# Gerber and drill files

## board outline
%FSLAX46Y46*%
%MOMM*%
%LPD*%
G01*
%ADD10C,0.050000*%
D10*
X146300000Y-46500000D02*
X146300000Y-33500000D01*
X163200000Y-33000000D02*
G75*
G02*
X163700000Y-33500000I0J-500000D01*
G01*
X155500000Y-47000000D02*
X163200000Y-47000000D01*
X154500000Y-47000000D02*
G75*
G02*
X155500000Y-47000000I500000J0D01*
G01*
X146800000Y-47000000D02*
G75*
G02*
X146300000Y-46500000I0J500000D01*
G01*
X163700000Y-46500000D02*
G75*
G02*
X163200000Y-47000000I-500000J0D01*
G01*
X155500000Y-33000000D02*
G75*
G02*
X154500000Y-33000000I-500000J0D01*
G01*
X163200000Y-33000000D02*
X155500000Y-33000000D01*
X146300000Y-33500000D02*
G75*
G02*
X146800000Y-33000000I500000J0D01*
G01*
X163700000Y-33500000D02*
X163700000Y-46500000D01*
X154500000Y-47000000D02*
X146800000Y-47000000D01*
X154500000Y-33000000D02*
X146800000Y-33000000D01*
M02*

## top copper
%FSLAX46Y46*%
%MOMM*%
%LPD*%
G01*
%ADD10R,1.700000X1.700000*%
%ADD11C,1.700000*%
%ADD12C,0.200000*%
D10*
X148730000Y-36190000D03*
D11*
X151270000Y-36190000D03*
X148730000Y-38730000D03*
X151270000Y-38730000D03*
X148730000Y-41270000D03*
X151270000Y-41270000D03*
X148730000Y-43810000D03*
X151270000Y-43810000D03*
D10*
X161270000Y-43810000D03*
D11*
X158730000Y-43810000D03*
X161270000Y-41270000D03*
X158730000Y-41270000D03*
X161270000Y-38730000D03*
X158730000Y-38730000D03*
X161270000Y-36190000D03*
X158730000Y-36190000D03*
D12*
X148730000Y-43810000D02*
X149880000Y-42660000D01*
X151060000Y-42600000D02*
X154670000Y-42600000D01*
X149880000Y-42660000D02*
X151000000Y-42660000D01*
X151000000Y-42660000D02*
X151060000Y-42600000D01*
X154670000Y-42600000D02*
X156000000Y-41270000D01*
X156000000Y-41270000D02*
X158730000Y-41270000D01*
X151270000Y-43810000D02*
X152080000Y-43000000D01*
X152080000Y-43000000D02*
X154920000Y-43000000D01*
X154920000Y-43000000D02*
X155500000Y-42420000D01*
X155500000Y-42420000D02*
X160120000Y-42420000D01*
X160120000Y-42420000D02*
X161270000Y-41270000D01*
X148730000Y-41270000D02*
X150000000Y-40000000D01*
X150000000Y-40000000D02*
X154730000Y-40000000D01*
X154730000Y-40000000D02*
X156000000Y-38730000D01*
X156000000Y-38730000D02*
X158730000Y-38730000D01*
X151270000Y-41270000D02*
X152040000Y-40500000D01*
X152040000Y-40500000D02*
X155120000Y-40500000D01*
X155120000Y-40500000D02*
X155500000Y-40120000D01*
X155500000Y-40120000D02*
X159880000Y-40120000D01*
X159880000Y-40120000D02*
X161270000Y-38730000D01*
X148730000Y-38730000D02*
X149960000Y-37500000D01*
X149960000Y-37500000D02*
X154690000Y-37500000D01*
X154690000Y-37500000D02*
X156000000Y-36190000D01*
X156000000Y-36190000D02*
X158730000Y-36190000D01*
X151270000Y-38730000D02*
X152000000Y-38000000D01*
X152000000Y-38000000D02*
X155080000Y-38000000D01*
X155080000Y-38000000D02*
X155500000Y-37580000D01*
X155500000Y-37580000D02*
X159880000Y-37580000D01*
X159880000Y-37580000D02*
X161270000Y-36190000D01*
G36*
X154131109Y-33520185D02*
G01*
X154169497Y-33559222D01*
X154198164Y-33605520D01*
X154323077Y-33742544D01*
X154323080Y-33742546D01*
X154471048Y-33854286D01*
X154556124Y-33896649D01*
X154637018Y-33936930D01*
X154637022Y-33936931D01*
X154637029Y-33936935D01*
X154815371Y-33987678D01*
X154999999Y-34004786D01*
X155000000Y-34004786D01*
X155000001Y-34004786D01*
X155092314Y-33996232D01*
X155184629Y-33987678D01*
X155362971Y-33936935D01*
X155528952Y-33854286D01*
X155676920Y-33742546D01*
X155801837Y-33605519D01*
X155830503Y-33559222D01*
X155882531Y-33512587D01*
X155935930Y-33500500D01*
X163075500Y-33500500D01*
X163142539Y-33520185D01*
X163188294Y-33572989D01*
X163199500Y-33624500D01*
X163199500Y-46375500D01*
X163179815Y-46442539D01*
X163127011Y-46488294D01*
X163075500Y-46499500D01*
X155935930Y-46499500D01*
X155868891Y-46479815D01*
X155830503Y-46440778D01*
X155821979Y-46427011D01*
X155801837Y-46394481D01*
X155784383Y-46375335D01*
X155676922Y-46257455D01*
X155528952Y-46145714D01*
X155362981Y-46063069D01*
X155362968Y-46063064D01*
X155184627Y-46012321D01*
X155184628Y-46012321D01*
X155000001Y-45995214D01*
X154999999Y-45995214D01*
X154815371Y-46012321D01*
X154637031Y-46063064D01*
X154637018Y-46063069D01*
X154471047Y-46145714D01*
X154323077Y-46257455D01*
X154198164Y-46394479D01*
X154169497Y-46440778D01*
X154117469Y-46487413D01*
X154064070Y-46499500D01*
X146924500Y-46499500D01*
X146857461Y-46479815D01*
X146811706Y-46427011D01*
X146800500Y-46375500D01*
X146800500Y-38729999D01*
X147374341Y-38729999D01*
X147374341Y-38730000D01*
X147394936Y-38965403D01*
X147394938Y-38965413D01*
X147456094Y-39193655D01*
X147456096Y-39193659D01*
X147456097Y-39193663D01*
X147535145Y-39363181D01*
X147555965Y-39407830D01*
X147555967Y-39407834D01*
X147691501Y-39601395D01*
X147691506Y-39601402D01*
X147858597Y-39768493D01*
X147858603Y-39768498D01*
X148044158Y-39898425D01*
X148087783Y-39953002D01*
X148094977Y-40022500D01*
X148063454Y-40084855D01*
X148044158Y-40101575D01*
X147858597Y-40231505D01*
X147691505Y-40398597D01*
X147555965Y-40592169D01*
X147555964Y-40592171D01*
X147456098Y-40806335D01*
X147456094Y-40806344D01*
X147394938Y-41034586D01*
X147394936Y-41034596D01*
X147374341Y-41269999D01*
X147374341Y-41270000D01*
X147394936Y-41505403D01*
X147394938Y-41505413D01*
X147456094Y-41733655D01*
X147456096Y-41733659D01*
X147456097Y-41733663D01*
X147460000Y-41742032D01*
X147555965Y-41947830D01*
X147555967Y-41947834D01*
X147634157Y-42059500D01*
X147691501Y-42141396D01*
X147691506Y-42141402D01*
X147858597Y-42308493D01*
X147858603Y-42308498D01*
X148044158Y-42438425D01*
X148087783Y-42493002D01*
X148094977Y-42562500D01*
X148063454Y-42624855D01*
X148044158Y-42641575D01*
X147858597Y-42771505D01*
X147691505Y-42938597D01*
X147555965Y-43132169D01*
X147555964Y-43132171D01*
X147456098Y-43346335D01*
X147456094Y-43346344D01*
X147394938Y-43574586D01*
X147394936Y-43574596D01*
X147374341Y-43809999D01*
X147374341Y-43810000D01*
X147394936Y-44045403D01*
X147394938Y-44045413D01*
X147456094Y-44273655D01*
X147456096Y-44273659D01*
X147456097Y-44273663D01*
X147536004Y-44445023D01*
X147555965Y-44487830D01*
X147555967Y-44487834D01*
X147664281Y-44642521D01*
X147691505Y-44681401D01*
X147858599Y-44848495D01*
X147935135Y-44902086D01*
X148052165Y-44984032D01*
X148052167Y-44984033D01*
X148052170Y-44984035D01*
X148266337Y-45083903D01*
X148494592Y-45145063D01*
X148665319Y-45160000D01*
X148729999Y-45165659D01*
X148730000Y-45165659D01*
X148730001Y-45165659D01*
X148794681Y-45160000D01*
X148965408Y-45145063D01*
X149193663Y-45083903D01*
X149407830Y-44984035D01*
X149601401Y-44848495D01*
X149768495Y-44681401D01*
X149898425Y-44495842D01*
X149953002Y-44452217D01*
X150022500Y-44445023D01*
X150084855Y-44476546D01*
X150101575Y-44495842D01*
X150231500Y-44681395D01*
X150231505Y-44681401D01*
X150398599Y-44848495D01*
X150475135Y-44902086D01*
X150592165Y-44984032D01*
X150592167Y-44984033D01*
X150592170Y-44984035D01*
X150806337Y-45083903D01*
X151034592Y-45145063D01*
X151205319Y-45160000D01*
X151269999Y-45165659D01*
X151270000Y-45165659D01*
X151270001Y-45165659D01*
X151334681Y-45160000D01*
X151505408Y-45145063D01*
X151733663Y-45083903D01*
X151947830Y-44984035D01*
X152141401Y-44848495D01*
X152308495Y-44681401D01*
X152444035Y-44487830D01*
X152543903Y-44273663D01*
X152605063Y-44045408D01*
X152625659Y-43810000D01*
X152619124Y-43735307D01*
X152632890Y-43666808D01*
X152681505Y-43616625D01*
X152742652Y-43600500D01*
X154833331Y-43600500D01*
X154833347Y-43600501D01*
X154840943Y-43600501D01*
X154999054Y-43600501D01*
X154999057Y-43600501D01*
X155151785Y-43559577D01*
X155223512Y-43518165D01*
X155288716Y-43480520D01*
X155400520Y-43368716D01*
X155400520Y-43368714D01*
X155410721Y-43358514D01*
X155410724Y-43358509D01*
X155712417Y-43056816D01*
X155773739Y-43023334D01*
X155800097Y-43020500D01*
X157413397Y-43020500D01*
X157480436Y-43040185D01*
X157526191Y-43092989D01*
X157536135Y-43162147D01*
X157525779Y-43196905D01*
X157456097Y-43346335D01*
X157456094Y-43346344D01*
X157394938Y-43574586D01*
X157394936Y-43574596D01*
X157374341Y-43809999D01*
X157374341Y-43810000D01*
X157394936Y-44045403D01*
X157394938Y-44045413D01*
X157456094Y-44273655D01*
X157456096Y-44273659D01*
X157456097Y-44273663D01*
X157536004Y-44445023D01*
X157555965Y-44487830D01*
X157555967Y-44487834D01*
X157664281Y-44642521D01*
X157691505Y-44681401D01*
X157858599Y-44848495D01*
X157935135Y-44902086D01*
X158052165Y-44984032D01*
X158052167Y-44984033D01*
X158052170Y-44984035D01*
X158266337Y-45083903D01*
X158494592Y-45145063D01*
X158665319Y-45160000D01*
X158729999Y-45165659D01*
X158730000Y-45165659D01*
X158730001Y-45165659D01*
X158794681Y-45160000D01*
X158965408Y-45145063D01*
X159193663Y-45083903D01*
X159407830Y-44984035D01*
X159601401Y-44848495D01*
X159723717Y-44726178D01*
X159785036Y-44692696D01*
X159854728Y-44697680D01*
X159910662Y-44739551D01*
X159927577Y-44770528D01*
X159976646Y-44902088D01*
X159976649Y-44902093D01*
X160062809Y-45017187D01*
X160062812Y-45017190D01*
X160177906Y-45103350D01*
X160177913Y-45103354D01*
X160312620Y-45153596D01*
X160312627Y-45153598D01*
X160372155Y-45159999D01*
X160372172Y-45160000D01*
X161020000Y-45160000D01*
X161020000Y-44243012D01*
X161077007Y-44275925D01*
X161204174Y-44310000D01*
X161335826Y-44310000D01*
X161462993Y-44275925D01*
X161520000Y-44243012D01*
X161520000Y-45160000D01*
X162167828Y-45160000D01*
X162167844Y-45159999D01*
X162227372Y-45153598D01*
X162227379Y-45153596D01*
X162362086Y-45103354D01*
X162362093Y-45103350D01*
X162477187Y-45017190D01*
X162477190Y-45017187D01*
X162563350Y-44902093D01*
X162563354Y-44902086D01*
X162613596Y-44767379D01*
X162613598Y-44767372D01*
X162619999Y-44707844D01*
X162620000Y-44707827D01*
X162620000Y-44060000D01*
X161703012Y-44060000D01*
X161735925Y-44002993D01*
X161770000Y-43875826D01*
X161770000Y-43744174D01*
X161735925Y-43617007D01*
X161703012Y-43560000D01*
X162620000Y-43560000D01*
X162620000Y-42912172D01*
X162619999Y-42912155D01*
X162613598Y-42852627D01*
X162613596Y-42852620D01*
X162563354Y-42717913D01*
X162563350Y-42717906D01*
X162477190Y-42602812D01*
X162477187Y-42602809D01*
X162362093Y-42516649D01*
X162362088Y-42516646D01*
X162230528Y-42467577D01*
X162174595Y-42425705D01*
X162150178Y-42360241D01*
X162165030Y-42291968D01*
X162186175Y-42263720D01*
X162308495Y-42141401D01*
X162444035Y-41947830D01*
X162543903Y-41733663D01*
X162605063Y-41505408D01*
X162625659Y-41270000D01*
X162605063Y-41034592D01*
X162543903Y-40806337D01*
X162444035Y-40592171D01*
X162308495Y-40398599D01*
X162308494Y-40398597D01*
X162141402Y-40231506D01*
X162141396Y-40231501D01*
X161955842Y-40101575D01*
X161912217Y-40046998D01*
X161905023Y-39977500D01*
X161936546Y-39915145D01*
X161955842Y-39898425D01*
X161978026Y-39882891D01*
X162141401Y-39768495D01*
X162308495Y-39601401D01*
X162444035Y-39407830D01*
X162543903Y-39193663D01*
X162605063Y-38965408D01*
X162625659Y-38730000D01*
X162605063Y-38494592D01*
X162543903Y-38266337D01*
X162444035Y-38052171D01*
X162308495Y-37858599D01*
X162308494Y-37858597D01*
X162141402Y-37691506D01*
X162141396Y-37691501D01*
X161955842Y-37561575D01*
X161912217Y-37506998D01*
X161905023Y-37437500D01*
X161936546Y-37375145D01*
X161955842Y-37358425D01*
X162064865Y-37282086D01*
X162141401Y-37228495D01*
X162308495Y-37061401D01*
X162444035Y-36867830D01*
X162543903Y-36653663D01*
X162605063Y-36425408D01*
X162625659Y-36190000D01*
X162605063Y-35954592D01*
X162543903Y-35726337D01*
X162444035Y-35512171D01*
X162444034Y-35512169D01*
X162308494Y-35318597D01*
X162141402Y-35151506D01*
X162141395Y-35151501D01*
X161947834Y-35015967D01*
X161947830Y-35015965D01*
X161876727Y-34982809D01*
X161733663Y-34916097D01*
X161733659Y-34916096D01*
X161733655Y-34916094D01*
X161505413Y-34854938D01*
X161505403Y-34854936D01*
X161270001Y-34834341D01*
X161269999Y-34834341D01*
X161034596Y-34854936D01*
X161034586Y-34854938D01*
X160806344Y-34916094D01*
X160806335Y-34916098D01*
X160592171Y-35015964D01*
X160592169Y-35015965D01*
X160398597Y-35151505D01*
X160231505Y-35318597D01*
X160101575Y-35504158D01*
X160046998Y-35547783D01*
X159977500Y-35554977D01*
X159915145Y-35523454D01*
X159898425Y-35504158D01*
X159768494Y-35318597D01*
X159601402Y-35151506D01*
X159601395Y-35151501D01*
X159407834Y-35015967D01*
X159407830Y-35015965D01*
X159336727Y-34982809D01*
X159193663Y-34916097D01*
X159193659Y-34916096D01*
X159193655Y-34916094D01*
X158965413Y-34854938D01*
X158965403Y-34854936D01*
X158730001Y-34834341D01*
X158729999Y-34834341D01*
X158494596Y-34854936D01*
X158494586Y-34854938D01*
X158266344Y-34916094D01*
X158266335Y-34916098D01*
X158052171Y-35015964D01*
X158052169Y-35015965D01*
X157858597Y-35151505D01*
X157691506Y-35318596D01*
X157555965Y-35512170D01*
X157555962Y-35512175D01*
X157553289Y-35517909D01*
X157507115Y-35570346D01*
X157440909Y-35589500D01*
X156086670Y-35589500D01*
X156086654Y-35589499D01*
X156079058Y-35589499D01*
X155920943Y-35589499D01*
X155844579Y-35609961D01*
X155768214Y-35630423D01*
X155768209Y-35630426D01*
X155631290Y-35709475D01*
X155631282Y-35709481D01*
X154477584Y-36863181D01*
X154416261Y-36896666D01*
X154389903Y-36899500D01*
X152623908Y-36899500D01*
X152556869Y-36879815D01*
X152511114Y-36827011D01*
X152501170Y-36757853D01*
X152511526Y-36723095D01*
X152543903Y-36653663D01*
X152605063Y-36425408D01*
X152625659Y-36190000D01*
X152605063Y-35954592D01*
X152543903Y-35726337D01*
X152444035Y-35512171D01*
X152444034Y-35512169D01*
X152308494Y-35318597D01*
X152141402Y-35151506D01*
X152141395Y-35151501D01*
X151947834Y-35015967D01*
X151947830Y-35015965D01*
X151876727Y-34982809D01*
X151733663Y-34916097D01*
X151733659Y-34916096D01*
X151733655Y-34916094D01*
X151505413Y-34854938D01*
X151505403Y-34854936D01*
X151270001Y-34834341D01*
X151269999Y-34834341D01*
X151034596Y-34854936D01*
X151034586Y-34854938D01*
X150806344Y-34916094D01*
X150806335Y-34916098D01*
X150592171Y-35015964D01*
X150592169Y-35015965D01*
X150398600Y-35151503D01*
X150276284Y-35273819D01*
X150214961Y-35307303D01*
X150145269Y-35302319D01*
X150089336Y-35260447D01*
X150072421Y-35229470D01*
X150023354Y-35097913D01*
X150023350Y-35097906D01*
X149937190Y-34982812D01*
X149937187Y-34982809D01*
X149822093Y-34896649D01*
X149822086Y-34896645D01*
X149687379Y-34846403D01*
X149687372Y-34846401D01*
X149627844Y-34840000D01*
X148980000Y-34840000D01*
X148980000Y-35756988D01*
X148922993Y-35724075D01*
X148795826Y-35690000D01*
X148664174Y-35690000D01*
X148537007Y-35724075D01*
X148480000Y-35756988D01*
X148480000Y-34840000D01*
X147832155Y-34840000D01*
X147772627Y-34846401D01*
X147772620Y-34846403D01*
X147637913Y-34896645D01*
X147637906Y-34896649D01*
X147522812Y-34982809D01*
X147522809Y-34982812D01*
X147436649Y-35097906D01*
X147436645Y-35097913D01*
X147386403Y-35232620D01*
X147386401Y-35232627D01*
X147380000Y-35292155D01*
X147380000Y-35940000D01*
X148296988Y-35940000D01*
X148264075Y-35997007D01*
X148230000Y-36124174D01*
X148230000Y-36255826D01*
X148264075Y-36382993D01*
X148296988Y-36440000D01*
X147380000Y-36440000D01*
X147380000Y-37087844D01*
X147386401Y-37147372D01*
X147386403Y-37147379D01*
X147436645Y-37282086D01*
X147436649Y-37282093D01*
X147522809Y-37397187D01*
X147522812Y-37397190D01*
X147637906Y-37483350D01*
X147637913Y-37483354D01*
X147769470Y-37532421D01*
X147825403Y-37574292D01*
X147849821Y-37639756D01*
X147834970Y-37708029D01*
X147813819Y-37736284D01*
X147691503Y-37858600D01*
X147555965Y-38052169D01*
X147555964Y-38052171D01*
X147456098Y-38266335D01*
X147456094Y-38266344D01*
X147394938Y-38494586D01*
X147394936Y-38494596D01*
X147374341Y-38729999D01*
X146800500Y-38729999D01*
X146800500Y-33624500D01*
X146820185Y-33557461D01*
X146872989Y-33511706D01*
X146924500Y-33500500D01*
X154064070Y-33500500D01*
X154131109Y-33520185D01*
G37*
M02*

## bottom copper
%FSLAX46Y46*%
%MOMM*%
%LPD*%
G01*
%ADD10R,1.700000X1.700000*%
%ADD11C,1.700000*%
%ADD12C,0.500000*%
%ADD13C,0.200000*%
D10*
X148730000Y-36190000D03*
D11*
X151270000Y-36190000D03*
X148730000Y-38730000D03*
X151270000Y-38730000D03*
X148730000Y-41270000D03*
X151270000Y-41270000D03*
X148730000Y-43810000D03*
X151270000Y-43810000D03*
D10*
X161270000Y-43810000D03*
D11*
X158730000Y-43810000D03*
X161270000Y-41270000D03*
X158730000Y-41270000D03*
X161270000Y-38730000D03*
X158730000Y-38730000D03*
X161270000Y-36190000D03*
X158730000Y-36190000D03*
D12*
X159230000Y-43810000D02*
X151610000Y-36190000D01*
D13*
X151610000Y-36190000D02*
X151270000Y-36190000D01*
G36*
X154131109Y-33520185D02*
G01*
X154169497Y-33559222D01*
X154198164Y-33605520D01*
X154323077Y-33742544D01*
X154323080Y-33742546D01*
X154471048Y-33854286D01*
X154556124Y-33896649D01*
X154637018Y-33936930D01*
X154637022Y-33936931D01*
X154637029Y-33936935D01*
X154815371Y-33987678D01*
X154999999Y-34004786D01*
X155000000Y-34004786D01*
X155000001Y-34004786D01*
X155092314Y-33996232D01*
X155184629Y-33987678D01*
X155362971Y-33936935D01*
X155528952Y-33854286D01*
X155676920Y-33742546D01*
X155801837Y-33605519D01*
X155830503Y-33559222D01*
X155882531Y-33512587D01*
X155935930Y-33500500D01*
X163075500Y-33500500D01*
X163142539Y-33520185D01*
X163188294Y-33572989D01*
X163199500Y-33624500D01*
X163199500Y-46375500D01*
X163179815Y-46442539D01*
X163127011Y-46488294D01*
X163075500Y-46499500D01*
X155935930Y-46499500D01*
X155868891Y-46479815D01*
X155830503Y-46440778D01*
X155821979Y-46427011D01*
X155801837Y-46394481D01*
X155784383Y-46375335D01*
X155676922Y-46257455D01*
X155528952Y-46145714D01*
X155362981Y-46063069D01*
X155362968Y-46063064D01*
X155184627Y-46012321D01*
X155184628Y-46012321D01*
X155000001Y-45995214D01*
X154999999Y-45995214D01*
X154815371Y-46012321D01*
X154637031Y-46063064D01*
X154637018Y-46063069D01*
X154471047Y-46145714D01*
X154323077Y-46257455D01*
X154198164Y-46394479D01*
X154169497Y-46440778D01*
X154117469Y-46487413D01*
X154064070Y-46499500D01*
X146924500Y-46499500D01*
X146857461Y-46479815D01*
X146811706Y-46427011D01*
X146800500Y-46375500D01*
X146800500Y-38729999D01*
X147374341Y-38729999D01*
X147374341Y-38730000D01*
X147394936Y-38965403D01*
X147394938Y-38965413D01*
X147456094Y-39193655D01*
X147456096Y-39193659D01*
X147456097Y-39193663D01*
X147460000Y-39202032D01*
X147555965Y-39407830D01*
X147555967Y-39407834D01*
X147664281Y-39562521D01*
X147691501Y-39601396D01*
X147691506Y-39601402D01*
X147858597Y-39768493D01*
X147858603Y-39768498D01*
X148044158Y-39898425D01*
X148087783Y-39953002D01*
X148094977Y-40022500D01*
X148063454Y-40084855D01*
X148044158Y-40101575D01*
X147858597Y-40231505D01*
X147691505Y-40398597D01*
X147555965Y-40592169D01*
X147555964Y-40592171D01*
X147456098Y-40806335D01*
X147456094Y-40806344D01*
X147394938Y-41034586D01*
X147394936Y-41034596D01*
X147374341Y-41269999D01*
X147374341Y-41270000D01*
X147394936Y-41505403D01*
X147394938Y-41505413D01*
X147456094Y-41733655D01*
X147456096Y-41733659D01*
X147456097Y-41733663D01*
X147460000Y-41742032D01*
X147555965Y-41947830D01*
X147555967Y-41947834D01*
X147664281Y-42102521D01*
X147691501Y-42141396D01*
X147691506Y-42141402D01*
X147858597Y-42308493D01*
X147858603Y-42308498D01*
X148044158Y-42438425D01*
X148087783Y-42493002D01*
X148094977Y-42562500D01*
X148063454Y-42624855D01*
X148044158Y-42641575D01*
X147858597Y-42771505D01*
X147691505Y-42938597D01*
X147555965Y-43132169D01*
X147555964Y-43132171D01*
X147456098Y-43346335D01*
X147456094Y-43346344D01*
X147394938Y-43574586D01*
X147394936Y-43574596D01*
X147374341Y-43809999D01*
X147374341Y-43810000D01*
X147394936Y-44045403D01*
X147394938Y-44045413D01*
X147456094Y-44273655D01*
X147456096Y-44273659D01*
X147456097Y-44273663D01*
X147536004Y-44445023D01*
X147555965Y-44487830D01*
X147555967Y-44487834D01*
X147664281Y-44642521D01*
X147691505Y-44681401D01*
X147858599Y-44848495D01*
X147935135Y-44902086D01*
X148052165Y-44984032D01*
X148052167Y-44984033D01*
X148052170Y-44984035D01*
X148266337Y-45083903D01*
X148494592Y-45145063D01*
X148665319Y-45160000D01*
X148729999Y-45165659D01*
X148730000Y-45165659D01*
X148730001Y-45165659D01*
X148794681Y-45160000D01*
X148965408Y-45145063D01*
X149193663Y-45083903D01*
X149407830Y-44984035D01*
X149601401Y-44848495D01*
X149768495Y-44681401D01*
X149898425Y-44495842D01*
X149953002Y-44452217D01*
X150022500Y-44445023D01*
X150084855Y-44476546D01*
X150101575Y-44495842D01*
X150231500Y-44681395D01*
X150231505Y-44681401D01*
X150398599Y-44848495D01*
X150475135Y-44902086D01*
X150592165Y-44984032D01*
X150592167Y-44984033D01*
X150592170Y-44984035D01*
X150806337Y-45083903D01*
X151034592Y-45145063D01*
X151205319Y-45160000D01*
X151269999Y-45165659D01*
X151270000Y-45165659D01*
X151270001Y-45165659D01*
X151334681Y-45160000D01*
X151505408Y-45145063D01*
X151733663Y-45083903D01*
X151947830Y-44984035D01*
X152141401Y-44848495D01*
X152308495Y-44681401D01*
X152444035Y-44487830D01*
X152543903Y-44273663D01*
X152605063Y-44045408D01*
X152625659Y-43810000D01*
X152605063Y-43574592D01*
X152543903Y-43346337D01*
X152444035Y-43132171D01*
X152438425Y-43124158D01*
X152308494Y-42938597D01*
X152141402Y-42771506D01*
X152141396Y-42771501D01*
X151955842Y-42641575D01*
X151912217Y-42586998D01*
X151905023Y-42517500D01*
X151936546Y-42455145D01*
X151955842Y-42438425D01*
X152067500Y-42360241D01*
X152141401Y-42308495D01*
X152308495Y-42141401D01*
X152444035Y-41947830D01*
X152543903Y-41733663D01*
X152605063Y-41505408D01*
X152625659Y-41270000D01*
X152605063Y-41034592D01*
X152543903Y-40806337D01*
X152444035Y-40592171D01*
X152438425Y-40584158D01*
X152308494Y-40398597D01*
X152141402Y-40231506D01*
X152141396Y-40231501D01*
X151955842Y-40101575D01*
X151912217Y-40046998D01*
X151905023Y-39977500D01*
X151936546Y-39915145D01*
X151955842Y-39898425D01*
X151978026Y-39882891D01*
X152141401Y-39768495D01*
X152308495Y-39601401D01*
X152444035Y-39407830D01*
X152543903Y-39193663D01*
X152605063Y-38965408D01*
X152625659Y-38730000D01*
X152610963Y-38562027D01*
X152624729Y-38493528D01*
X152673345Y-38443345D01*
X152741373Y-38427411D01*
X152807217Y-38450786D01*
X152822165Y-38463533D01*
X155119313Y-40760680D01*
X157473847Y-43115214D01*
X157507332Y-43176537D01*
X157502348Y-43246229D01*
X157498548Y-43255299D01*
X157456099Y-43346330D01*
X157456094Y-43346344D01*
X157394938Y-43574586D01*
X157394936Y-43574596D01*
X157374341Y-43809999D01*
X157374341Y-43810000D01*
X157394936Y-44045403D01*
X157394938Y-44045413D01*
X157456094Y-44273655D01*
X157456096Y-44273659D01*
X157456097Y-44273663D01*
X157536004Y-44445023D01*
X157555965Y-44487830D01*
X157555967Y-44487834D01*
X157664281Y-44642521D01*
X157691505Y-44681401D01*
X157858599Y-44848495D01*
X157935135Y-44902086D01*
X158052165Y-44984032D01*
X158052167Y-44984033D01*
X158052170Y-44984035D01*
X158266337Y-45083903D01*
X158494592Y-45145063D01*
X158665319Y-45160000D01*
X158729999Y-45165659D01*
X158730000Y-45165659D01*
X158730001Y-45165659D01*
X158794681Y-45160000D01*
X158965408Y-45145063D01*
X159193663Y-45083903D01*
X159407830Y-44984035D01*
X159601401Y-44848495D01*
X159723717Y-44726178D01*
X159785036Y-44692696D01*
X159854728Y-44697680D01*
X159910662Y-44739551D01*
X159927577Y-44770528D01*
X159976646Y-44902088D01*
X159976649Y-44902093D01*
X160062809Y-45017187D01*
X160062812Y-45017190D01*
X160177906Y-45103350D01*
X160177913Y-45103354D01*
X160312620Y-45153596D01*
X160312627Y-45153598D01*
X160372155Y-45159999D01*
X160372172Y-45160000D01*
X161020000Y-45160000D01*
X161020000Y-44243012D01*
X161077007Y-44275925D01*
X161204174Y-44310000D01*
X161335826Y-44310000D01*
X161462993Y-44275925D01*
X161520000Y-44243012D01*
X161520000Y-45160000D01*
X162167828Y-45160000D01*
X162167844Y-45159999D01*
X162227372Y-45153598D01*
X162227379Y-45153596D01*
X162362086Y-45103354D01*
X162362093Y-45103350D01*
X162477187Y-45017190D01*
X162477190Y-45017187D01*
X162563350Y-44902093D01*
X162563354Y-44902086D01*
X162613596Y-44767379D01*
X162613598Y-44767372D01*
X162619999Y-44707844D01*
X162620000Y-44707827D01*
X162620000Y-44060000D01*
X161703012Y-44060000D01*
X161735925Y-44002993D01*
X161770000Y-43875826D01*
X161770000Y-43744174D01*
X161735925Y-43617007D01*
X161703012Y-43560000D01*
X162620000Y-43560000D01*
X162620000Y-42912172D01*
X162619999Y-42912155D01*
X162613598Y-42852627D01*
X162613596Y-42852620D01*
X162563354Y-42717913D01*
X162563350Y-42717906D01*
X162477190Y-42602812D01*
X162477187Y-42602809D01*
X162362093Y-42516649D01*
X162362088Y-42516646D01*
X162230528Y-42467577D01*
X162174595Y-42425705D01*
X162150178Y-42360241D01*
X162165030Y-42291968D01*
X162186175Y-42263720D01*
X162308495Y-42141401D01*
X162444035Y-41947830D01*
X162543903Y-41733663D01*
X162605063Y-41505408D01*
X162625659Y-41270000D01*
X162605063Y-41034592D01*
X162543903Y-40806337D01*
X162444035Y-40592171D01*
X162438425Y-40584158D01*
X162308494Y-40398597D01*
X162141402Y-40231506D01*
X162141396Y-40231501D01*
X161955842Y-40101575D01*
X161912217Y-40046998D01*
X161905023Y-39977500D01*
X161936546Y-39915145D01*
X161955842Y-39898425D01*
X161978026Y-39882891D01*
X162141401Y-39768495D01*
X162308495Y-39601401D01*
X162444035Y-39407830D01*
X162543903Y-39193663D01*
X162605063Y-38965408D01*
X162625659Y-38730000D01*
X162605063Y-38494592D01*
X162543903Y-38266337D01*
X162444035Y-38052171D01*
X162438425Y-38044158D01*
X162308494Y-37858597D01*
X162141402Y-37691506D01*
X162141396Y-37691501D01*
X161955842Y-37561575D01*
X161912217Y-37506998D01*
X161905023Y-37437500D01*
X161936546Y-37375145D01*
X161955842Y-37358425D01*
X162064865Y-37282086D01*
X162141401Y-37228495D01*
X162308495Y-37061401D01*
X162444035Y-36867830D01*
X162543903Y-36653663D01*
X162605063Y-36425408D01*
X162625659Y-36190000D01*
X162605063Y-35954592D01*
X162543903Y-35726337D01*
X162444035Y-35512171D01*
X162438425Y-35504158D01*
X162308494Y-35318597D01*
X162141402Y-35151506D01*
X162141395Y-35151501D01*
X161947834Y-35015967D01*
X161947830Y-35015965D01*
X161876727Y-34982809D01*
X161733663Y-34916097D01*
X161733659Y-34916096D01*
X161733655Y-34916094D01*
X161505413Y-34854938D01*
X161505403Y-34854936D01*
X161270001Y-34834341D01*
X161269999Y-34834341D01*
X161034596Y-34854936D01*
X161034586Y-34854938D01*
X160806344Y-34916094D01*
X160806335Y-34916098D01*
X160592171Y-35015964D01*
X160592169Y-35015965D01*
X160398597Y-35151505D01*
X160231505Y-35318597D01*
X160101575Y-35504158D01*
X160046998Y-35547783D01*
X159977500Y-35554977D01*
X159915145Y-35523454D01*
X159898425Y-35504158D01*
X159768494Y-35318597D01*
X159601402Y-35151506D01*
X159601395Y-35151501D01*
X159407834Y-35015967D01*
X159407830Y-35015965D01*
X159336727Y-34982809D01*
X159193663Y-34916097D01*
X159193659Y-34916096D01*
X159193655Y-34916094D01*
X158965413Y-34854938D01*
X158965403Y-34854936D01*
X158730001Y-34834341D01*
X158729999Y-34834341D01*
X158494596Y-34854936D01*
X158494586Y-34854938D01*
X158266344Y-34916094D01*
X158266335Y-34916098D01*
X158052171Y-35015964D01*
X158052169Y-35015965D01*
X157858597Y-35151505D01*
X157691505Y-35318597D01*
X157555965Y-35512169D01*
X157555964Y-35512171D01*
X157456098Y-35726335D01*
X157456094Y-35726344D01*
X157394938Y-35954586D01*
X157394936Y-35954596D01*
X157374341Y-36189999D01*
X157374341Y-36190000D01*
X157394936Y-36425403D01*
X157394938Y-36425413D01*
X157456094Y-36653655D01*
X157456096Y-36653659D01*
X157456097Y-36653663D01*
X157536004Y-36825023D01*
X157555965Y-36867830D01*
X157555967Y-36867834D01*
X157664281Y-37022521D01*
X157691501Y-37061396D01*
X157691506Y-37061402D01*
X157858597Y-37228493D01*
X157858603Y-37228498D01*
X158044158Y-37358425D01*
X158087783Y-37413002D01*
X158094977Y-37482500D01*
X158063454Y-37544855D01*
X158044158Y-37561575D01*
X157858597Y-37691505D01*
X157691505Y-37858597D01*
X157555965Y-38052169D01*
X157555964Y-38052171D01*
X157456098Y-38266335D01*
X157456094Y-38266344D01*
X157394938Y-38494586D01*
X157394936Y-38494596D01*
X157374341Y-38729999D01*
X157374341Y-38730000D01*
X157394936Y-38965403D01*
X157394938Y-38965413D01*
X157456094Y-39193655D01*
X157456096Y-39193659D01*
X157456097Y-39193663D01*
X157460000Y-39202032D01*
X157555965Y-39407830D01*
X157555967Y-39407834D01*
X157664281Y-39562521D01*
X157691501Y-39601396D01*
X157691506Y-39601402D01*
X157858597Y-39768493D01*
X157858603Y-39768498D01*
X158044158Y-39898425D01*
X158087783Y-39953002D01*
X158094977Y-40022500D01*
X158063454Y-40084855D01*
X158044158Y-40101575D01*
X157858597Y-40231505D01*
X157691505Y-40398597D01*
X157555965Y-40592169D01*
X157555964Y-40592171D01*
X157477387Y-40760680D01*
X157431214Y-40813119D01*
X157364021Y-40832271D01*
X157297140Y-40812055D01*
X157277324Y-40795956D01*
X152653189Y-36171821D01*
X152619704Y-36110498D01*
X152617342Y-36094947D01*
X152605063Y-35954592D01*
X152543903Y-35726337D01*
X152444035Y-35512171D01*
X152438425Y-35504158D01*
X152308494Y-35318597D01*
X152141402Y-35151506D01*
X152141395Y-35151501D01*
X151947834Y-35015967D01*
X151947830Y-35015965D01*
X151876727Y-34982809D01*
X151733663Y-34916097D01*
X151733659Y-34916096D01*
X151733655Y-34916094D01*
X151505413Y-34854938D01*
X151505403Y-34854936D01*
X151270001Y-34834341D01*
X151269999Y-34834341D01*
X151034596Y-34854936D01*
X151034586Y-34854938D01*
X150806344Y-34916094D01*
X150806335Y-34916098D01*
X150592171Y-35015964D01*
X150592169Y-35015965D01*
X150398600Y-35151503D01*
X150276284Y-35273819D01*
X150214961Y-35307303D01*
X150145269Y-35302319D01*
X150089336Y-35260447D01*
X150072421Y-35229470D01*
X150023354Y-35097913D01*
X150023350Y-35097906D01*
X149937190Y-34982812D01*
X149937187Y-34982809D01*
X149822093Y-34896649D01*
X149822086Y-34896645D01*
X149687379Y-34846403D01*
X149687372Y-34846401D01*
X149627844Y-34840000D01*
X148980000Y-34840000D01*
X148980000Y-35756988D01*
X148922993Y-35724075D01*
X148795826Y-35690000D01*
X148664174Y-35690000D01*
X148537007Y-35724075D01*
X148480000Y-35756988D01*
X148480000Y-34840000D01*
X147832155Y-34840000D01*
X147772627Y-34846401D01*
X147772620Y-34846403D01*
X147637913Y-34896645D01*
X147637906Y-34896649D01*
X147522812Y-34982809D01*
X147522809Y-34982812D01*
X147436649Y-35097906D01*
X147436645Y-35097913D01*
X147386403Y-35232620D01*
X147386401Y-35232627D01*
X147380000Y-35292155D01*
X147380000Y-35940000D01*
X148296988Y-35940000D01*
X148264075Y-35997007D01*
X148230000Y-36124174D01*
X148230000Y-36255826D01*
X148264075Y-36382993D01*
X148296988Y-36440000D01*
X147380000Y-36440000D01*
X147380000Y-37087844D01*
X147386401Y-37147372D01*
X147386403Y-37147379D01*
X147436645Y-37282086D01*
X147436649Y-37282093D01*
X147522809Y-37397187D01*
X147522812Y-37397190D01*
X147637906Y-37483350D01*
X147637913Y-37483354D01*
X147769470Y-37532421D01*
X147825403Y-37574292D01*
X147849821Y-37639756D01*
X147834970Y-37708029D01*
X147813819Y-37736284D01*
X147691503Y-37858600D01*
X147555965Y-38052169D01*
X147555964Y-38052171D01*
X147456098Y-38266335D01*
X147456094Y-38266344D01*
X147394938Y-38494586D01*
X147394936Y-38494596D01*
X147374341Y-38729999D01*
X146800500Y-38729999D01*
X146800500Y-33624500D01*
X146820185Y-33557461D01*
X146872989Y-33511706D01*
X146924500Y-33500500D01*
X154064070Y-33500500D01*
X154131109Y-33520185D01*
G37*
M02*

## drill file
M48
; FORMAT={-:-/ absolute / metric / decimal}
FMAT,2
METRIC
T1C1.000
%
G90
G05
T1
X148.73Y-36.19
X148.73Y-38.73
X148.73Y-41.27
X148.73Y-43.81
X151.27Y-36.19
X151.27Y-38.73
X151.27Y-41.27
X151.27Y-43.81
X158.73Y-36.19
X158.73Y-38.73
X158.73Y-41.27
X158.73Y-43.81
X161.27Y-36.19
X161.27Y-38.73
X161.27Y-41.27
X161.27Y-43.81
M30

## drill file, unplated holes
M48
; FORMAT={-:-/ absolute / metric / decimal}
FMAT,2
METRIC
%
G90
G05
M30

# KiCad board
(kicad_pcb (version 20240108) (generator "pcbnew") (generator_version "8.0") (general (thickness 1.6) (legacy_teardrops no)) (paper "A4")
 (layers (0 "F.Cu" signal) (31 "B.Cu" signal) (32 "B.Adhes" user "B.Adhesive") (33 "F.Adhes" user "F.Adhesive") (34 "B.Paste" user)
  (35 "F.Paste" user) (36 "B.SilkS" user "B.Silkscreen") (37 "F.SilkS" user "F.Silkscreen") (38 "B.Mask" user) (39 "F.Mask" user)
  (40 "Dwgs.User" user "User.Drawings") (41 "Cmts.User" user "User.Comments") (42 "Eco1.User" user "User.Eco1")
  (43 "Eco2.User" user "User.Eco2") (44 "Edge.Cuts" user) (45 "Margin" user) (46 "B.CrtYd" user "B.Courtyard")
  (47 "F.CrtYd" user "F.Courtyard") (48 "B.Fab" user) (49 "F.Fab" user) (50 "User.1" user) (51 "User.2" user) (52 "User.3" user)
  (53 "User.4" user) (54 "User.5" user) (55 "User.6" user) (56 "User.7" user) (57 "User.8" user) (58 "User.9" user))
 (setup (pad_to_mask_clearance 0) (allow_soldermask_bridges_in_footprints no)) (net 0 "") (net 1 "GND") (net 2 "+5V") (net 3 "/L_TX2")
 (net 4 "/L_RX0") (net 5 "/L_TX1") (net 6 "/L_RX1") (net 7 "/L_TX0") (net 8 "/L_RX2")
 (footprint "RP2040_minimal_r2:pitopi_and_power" (layer "F.Cu") (at 150 40 180)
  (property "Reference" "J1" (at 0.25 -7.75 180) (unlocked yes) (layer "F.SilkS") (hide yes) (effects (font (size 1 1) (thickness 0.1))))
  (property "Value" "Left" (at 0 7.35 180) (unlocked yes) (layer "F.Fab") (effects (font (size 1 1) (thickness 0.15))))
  (pad "1" thru_hole rect (at 1.27 3.81 180) (size 1.7 1.7) (drill 1) (layers "*.Cu" "*.Mask") (remove_unused_layers no) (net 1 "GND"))
  (pad "2" thru_hole circle (at -1.27 3.81 180) (size 1.7 1.7) (drill 1) (layers "*.Cu" "*.Mask") (remove_unused_layers no) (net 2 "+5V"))
  (pad "3" thru_hole circle (at 1.27 1.27 180) (size 1.7 1.7) (drill 1) (layers "*.Cu" "*.Mask") (remove_unused_layers no) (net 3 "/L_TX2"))
  (pad "4" thru_hole circle (at -1.27 1.27 180) (size 1.7 1.7) (drill 1) (layers "*.Cu" "*.Mask") (remove_unused_layers no) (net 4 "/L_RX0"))
  (pad "5" thru_hole circle (at 1.27 -1.27 180) (size 1.7 1.7) (drill 1) (layers "*.Cu" "*.Mask") (remove_unused_layers no) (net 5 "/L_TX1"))
  (pad "6" thru_hole circle (at -1.27 -1.27 180) (size 1.7 1.7) (drill 1) (layers "*.Cu" "*.Mask") (remove_unused_layers no)
   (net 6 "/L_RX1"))
  (pad "7" thru_hole circle (at 1.27 -3.81 180) (size 1.7 1.7) (drill 1) (layers "*.Cu" "*.Mask") (remove_unused_layers no) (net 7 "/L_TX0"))
  (pad "8" thru_hole circle (at -1.27 -3.81 180) (size 1.7 1.7) (drill 1) (layers "*.Cu" "*.Mask") (remove_unused_layers no)
   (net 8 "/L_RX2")))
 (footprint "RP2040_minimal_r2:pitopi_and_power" (layer "F.Cu") (at 160 40)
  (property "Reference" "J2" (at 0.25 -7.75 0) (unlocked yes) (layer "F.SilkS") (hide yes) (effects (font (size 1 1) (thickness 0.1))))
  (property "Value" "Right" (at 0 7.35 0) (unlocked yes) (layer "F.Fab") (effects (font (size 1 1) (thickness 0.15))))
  (pad "1" thru_hole rect (at 1.27 3.81) (size 1.7 1.7) (drill 1) (layers "*.Cu" "*.Mask") (remove_unused_layers no) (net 1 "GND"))
  (pad "2" thru_hole circle (at -1.27 3.81) (size 1.7 1.7) (drill 1) (layers "*.Cu" "*.Mask") (remove_unused_layers no) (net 2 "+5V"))
  (pad "3" thru_hole circle (at 1.27 1.27) (size 1.7 1.7) (drill 1) (layers "*.Cu" "*.Mask") (remove_unused_layers no) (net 8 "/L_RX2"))
  (pad "4" thru_hole circle (at -1.27 1.27) (size 1.7 1.7) (drill 1) (layers "*.Cu" "*.Mask") (remove_unused_layers no) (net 7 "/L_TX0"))
  (pad "5" thru_hole circle (at 1.27 -1.27) (size 1.7 1.7) (drill 1) (layers "*.Cu" "*.Mask") (remove_unused_layers no) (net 6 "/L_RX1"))
  (pad "6" thru_hole circle (at -1.27 -1.27) (size 1.7 1.7) (drill 1) (layers "*.Cu" "*.Mask") (remove_unused_layers no) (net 5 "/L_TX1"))
  (pad "7" thru_hole circle (at 1.27 -3.81) (size 1.7 1.7) (drill 1) (layers "*.Cu" "*.Mask") (remove_unused_layers no) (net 4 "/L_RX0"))
  (pad "8" thru_hole circle (at -1.27 -3.81) (size 1.7 1.7) (drill 1) (layers "*.Cu" "*.Mask") (remove_unused_layers no) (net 3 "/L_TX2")))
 (gr_line (start 146.3 46.5) (end 146.3 33.5) (stroke (width 0.05) (type default)) (layer "Edge.Cuts"))
 (gr_arc (start 163.2 33) (mid 163.553553 33.146447) (end 163.7 33.5) (stroke (width 0.05) (type default)) (layer "Edge.Cuts"))
 (gr_line (start 155.5 47) (end 163.2 47) (stroke (width 0.05) (type default)) (layer "Edge.Cuts"))
 (gr_arc (start 154.5 47) (mid 155 46.5) (end 155.5 47) (stroke (width 0.05) (type default)) (layer "Edge.Cuts"))
 (gr_arc (start 146.8 47) (mid 146.446447 46.853553) (end 146.3 46.5) (stroke (width 0.05) (type default)) (layer "Edge.Cuts"))
 (gr_arc (start 163.7 46.5) (mid 163.553553 46.853553) (end 163.2 47) (stroke (width 0.05) (type default)) (layer "Edge.Cuts"))
 (gr_arc (start 155.5 33) (mid 155 33.5) (end 154.5 33) (stroke (width 0.05) (type default)) (layer "Edge.Cuts"))
 (gr_line (start 163.2 33) (end 155.5 33) (stroke (width 0.05) (type default)) (layer "Edge.Cuts"))
 (gr_arc (start 146.3 33.5) (mid 146.446447 33.146447) (end 146.8 33) (stroke (width 0.05) (type default)) (layer "Edge.Cuts"))
 (gr_line (start 163.7 33.5) (end 163.7 46.5) (stroke (width 0.05) (type default)) (layer "Edge.Cuts"))
 (gr_line (start 154.5 47) (end 146.8 47) (stroke (width 0.05) (type default)) (layer "Edge.Cuts"))
 (gr_line (start 154.5 33) (end 146.8 33) (stroke (width 0.05) (type default)) (layer "Edge.Cuts"))
 (segment (start 155.5 42.42) (end 160.12 42.42) (width 0.2) (layer "F.Cu") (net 8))
 (segment (start 160.12 42.42) (end 161.27 41.27) (width 0.2) (layer "F.Cu") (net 8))
 (segment (start 154.92 43) (end 155.5 42.42) (width 0.2) (layer "F.Cu") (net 8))
 (segment (start 151.27 43.81) (end 152.08 43) (width 0.2) (layer "F.Cu") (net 8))
 (segment (start 152.08 43) (end 154.92 43) (width 0.2) (layer "F.Cu") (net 8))
 (segment (start 148.73 41.27) (end 150 40) (width 0.2) (layer "F.Cu") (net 5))
 (segment (start 150 40) (end 154.73 40) (width 0.2) (layer "F.Cu") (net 5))
 (segment (start 154.73 40) (end 156 38.73) (width 0.2) (layer "F.Cu") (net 5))
 (segment (start 156 38.73) (end 158.73 38.73) (width 0.2) (layer "F.Cu") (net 5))
 (segment (start 151.27 41.27) (end 152.04 40.5) (width 0.2) (layer "F.Cu") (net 6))
 (segment (start 152.04 40.5) (end 155.12 40.5) (width 0.2) (layer "F.Cu") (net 6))
 (segment (start 159.88 40.12) (end 161.27 38.73) (width 0.2) (layer "F.Cu") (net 6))
 (segment (start 155.5 40.12) (end 159.88 40.12) (width 0.2) (layer "F.Cu") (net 6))
 (segment (start 155.12 40.5) (end 155.5 40.12) (width 0.2) (layer "F.Cu") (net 6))
 (segment (start 156 36.19) (end 158.73 36.19) (width 0.2) (layer "F.Cu") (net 3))
 (segment (start 149.96 37.5) (end 154.69 37.5) (width 0.2) (layer "F.Cu") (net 3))
 (segment (start 154.69 37.5) (end 156 36.19) (width 0.2) (layer "F.Cu") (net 3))
 (segment (start 148.73 38.73) (end 149.96 37.5) (width 0.2) (layer "F.Cu") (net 3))
 (segment (start 154.67 42.6) (end 156 41.27) (width 0.2) (layer "F.Cu") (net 7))
 (segment (start 148.73 43.81) (end 149.88 42.66) (width 0.2) (layer "F.Cu") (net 7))
 (segment (start 151 42.66) (end 151.06 42.6) (width 0.2) (layer "F.Cu") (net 7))
 (segment (start 149.88 42.66) (end 151 42.66) (width 0.2) (layer "F.Cu") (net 7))
 (segment (start 151.06 42.6) (end 154.67 42.6) (width 0.2) (layer "F.Cu") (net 7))
 (segment (start 156 41.27) (end 158.73 41.27) (width 0.2) (layer "F.Cu") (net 7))
 (segment (start 155.08 38) (end 155.5 37.58) (width 0.2) (layer "F.Cu") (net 4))
 (segment (start 151.27 38.73) (end 152 38) (width 0.2) (layer "F.Cu") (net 4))
 (segment (start 155.5 37.58) (end 159.88 37.58) (width 0.2) (layer "F.Cu") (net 4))
 (segment (start 159.88 37.58) (end 161.27 36.19) (width 0.2) (layer "F.Cu") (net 4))
 (segment (start 152 38) (end 155.08 38) (width 0.2) (layer "F.Cu") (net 4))
 (segment (start 159.23 43.81) (end 151.61 36.19) (width 0.5) (layer "B.Cu") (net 2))
 (segment (start 151.61 36.19) (end 151.27 36.19) (width 0.2) (layer "B.Cu") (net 2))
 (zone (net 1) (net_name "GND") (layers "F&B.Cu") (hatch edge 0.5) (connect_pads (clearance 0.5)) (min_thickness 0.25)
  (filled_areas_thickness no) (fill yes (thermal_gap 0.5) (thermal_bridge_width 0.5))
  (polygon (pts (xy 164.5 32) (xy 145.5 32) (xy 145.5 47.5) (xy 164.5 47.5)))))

